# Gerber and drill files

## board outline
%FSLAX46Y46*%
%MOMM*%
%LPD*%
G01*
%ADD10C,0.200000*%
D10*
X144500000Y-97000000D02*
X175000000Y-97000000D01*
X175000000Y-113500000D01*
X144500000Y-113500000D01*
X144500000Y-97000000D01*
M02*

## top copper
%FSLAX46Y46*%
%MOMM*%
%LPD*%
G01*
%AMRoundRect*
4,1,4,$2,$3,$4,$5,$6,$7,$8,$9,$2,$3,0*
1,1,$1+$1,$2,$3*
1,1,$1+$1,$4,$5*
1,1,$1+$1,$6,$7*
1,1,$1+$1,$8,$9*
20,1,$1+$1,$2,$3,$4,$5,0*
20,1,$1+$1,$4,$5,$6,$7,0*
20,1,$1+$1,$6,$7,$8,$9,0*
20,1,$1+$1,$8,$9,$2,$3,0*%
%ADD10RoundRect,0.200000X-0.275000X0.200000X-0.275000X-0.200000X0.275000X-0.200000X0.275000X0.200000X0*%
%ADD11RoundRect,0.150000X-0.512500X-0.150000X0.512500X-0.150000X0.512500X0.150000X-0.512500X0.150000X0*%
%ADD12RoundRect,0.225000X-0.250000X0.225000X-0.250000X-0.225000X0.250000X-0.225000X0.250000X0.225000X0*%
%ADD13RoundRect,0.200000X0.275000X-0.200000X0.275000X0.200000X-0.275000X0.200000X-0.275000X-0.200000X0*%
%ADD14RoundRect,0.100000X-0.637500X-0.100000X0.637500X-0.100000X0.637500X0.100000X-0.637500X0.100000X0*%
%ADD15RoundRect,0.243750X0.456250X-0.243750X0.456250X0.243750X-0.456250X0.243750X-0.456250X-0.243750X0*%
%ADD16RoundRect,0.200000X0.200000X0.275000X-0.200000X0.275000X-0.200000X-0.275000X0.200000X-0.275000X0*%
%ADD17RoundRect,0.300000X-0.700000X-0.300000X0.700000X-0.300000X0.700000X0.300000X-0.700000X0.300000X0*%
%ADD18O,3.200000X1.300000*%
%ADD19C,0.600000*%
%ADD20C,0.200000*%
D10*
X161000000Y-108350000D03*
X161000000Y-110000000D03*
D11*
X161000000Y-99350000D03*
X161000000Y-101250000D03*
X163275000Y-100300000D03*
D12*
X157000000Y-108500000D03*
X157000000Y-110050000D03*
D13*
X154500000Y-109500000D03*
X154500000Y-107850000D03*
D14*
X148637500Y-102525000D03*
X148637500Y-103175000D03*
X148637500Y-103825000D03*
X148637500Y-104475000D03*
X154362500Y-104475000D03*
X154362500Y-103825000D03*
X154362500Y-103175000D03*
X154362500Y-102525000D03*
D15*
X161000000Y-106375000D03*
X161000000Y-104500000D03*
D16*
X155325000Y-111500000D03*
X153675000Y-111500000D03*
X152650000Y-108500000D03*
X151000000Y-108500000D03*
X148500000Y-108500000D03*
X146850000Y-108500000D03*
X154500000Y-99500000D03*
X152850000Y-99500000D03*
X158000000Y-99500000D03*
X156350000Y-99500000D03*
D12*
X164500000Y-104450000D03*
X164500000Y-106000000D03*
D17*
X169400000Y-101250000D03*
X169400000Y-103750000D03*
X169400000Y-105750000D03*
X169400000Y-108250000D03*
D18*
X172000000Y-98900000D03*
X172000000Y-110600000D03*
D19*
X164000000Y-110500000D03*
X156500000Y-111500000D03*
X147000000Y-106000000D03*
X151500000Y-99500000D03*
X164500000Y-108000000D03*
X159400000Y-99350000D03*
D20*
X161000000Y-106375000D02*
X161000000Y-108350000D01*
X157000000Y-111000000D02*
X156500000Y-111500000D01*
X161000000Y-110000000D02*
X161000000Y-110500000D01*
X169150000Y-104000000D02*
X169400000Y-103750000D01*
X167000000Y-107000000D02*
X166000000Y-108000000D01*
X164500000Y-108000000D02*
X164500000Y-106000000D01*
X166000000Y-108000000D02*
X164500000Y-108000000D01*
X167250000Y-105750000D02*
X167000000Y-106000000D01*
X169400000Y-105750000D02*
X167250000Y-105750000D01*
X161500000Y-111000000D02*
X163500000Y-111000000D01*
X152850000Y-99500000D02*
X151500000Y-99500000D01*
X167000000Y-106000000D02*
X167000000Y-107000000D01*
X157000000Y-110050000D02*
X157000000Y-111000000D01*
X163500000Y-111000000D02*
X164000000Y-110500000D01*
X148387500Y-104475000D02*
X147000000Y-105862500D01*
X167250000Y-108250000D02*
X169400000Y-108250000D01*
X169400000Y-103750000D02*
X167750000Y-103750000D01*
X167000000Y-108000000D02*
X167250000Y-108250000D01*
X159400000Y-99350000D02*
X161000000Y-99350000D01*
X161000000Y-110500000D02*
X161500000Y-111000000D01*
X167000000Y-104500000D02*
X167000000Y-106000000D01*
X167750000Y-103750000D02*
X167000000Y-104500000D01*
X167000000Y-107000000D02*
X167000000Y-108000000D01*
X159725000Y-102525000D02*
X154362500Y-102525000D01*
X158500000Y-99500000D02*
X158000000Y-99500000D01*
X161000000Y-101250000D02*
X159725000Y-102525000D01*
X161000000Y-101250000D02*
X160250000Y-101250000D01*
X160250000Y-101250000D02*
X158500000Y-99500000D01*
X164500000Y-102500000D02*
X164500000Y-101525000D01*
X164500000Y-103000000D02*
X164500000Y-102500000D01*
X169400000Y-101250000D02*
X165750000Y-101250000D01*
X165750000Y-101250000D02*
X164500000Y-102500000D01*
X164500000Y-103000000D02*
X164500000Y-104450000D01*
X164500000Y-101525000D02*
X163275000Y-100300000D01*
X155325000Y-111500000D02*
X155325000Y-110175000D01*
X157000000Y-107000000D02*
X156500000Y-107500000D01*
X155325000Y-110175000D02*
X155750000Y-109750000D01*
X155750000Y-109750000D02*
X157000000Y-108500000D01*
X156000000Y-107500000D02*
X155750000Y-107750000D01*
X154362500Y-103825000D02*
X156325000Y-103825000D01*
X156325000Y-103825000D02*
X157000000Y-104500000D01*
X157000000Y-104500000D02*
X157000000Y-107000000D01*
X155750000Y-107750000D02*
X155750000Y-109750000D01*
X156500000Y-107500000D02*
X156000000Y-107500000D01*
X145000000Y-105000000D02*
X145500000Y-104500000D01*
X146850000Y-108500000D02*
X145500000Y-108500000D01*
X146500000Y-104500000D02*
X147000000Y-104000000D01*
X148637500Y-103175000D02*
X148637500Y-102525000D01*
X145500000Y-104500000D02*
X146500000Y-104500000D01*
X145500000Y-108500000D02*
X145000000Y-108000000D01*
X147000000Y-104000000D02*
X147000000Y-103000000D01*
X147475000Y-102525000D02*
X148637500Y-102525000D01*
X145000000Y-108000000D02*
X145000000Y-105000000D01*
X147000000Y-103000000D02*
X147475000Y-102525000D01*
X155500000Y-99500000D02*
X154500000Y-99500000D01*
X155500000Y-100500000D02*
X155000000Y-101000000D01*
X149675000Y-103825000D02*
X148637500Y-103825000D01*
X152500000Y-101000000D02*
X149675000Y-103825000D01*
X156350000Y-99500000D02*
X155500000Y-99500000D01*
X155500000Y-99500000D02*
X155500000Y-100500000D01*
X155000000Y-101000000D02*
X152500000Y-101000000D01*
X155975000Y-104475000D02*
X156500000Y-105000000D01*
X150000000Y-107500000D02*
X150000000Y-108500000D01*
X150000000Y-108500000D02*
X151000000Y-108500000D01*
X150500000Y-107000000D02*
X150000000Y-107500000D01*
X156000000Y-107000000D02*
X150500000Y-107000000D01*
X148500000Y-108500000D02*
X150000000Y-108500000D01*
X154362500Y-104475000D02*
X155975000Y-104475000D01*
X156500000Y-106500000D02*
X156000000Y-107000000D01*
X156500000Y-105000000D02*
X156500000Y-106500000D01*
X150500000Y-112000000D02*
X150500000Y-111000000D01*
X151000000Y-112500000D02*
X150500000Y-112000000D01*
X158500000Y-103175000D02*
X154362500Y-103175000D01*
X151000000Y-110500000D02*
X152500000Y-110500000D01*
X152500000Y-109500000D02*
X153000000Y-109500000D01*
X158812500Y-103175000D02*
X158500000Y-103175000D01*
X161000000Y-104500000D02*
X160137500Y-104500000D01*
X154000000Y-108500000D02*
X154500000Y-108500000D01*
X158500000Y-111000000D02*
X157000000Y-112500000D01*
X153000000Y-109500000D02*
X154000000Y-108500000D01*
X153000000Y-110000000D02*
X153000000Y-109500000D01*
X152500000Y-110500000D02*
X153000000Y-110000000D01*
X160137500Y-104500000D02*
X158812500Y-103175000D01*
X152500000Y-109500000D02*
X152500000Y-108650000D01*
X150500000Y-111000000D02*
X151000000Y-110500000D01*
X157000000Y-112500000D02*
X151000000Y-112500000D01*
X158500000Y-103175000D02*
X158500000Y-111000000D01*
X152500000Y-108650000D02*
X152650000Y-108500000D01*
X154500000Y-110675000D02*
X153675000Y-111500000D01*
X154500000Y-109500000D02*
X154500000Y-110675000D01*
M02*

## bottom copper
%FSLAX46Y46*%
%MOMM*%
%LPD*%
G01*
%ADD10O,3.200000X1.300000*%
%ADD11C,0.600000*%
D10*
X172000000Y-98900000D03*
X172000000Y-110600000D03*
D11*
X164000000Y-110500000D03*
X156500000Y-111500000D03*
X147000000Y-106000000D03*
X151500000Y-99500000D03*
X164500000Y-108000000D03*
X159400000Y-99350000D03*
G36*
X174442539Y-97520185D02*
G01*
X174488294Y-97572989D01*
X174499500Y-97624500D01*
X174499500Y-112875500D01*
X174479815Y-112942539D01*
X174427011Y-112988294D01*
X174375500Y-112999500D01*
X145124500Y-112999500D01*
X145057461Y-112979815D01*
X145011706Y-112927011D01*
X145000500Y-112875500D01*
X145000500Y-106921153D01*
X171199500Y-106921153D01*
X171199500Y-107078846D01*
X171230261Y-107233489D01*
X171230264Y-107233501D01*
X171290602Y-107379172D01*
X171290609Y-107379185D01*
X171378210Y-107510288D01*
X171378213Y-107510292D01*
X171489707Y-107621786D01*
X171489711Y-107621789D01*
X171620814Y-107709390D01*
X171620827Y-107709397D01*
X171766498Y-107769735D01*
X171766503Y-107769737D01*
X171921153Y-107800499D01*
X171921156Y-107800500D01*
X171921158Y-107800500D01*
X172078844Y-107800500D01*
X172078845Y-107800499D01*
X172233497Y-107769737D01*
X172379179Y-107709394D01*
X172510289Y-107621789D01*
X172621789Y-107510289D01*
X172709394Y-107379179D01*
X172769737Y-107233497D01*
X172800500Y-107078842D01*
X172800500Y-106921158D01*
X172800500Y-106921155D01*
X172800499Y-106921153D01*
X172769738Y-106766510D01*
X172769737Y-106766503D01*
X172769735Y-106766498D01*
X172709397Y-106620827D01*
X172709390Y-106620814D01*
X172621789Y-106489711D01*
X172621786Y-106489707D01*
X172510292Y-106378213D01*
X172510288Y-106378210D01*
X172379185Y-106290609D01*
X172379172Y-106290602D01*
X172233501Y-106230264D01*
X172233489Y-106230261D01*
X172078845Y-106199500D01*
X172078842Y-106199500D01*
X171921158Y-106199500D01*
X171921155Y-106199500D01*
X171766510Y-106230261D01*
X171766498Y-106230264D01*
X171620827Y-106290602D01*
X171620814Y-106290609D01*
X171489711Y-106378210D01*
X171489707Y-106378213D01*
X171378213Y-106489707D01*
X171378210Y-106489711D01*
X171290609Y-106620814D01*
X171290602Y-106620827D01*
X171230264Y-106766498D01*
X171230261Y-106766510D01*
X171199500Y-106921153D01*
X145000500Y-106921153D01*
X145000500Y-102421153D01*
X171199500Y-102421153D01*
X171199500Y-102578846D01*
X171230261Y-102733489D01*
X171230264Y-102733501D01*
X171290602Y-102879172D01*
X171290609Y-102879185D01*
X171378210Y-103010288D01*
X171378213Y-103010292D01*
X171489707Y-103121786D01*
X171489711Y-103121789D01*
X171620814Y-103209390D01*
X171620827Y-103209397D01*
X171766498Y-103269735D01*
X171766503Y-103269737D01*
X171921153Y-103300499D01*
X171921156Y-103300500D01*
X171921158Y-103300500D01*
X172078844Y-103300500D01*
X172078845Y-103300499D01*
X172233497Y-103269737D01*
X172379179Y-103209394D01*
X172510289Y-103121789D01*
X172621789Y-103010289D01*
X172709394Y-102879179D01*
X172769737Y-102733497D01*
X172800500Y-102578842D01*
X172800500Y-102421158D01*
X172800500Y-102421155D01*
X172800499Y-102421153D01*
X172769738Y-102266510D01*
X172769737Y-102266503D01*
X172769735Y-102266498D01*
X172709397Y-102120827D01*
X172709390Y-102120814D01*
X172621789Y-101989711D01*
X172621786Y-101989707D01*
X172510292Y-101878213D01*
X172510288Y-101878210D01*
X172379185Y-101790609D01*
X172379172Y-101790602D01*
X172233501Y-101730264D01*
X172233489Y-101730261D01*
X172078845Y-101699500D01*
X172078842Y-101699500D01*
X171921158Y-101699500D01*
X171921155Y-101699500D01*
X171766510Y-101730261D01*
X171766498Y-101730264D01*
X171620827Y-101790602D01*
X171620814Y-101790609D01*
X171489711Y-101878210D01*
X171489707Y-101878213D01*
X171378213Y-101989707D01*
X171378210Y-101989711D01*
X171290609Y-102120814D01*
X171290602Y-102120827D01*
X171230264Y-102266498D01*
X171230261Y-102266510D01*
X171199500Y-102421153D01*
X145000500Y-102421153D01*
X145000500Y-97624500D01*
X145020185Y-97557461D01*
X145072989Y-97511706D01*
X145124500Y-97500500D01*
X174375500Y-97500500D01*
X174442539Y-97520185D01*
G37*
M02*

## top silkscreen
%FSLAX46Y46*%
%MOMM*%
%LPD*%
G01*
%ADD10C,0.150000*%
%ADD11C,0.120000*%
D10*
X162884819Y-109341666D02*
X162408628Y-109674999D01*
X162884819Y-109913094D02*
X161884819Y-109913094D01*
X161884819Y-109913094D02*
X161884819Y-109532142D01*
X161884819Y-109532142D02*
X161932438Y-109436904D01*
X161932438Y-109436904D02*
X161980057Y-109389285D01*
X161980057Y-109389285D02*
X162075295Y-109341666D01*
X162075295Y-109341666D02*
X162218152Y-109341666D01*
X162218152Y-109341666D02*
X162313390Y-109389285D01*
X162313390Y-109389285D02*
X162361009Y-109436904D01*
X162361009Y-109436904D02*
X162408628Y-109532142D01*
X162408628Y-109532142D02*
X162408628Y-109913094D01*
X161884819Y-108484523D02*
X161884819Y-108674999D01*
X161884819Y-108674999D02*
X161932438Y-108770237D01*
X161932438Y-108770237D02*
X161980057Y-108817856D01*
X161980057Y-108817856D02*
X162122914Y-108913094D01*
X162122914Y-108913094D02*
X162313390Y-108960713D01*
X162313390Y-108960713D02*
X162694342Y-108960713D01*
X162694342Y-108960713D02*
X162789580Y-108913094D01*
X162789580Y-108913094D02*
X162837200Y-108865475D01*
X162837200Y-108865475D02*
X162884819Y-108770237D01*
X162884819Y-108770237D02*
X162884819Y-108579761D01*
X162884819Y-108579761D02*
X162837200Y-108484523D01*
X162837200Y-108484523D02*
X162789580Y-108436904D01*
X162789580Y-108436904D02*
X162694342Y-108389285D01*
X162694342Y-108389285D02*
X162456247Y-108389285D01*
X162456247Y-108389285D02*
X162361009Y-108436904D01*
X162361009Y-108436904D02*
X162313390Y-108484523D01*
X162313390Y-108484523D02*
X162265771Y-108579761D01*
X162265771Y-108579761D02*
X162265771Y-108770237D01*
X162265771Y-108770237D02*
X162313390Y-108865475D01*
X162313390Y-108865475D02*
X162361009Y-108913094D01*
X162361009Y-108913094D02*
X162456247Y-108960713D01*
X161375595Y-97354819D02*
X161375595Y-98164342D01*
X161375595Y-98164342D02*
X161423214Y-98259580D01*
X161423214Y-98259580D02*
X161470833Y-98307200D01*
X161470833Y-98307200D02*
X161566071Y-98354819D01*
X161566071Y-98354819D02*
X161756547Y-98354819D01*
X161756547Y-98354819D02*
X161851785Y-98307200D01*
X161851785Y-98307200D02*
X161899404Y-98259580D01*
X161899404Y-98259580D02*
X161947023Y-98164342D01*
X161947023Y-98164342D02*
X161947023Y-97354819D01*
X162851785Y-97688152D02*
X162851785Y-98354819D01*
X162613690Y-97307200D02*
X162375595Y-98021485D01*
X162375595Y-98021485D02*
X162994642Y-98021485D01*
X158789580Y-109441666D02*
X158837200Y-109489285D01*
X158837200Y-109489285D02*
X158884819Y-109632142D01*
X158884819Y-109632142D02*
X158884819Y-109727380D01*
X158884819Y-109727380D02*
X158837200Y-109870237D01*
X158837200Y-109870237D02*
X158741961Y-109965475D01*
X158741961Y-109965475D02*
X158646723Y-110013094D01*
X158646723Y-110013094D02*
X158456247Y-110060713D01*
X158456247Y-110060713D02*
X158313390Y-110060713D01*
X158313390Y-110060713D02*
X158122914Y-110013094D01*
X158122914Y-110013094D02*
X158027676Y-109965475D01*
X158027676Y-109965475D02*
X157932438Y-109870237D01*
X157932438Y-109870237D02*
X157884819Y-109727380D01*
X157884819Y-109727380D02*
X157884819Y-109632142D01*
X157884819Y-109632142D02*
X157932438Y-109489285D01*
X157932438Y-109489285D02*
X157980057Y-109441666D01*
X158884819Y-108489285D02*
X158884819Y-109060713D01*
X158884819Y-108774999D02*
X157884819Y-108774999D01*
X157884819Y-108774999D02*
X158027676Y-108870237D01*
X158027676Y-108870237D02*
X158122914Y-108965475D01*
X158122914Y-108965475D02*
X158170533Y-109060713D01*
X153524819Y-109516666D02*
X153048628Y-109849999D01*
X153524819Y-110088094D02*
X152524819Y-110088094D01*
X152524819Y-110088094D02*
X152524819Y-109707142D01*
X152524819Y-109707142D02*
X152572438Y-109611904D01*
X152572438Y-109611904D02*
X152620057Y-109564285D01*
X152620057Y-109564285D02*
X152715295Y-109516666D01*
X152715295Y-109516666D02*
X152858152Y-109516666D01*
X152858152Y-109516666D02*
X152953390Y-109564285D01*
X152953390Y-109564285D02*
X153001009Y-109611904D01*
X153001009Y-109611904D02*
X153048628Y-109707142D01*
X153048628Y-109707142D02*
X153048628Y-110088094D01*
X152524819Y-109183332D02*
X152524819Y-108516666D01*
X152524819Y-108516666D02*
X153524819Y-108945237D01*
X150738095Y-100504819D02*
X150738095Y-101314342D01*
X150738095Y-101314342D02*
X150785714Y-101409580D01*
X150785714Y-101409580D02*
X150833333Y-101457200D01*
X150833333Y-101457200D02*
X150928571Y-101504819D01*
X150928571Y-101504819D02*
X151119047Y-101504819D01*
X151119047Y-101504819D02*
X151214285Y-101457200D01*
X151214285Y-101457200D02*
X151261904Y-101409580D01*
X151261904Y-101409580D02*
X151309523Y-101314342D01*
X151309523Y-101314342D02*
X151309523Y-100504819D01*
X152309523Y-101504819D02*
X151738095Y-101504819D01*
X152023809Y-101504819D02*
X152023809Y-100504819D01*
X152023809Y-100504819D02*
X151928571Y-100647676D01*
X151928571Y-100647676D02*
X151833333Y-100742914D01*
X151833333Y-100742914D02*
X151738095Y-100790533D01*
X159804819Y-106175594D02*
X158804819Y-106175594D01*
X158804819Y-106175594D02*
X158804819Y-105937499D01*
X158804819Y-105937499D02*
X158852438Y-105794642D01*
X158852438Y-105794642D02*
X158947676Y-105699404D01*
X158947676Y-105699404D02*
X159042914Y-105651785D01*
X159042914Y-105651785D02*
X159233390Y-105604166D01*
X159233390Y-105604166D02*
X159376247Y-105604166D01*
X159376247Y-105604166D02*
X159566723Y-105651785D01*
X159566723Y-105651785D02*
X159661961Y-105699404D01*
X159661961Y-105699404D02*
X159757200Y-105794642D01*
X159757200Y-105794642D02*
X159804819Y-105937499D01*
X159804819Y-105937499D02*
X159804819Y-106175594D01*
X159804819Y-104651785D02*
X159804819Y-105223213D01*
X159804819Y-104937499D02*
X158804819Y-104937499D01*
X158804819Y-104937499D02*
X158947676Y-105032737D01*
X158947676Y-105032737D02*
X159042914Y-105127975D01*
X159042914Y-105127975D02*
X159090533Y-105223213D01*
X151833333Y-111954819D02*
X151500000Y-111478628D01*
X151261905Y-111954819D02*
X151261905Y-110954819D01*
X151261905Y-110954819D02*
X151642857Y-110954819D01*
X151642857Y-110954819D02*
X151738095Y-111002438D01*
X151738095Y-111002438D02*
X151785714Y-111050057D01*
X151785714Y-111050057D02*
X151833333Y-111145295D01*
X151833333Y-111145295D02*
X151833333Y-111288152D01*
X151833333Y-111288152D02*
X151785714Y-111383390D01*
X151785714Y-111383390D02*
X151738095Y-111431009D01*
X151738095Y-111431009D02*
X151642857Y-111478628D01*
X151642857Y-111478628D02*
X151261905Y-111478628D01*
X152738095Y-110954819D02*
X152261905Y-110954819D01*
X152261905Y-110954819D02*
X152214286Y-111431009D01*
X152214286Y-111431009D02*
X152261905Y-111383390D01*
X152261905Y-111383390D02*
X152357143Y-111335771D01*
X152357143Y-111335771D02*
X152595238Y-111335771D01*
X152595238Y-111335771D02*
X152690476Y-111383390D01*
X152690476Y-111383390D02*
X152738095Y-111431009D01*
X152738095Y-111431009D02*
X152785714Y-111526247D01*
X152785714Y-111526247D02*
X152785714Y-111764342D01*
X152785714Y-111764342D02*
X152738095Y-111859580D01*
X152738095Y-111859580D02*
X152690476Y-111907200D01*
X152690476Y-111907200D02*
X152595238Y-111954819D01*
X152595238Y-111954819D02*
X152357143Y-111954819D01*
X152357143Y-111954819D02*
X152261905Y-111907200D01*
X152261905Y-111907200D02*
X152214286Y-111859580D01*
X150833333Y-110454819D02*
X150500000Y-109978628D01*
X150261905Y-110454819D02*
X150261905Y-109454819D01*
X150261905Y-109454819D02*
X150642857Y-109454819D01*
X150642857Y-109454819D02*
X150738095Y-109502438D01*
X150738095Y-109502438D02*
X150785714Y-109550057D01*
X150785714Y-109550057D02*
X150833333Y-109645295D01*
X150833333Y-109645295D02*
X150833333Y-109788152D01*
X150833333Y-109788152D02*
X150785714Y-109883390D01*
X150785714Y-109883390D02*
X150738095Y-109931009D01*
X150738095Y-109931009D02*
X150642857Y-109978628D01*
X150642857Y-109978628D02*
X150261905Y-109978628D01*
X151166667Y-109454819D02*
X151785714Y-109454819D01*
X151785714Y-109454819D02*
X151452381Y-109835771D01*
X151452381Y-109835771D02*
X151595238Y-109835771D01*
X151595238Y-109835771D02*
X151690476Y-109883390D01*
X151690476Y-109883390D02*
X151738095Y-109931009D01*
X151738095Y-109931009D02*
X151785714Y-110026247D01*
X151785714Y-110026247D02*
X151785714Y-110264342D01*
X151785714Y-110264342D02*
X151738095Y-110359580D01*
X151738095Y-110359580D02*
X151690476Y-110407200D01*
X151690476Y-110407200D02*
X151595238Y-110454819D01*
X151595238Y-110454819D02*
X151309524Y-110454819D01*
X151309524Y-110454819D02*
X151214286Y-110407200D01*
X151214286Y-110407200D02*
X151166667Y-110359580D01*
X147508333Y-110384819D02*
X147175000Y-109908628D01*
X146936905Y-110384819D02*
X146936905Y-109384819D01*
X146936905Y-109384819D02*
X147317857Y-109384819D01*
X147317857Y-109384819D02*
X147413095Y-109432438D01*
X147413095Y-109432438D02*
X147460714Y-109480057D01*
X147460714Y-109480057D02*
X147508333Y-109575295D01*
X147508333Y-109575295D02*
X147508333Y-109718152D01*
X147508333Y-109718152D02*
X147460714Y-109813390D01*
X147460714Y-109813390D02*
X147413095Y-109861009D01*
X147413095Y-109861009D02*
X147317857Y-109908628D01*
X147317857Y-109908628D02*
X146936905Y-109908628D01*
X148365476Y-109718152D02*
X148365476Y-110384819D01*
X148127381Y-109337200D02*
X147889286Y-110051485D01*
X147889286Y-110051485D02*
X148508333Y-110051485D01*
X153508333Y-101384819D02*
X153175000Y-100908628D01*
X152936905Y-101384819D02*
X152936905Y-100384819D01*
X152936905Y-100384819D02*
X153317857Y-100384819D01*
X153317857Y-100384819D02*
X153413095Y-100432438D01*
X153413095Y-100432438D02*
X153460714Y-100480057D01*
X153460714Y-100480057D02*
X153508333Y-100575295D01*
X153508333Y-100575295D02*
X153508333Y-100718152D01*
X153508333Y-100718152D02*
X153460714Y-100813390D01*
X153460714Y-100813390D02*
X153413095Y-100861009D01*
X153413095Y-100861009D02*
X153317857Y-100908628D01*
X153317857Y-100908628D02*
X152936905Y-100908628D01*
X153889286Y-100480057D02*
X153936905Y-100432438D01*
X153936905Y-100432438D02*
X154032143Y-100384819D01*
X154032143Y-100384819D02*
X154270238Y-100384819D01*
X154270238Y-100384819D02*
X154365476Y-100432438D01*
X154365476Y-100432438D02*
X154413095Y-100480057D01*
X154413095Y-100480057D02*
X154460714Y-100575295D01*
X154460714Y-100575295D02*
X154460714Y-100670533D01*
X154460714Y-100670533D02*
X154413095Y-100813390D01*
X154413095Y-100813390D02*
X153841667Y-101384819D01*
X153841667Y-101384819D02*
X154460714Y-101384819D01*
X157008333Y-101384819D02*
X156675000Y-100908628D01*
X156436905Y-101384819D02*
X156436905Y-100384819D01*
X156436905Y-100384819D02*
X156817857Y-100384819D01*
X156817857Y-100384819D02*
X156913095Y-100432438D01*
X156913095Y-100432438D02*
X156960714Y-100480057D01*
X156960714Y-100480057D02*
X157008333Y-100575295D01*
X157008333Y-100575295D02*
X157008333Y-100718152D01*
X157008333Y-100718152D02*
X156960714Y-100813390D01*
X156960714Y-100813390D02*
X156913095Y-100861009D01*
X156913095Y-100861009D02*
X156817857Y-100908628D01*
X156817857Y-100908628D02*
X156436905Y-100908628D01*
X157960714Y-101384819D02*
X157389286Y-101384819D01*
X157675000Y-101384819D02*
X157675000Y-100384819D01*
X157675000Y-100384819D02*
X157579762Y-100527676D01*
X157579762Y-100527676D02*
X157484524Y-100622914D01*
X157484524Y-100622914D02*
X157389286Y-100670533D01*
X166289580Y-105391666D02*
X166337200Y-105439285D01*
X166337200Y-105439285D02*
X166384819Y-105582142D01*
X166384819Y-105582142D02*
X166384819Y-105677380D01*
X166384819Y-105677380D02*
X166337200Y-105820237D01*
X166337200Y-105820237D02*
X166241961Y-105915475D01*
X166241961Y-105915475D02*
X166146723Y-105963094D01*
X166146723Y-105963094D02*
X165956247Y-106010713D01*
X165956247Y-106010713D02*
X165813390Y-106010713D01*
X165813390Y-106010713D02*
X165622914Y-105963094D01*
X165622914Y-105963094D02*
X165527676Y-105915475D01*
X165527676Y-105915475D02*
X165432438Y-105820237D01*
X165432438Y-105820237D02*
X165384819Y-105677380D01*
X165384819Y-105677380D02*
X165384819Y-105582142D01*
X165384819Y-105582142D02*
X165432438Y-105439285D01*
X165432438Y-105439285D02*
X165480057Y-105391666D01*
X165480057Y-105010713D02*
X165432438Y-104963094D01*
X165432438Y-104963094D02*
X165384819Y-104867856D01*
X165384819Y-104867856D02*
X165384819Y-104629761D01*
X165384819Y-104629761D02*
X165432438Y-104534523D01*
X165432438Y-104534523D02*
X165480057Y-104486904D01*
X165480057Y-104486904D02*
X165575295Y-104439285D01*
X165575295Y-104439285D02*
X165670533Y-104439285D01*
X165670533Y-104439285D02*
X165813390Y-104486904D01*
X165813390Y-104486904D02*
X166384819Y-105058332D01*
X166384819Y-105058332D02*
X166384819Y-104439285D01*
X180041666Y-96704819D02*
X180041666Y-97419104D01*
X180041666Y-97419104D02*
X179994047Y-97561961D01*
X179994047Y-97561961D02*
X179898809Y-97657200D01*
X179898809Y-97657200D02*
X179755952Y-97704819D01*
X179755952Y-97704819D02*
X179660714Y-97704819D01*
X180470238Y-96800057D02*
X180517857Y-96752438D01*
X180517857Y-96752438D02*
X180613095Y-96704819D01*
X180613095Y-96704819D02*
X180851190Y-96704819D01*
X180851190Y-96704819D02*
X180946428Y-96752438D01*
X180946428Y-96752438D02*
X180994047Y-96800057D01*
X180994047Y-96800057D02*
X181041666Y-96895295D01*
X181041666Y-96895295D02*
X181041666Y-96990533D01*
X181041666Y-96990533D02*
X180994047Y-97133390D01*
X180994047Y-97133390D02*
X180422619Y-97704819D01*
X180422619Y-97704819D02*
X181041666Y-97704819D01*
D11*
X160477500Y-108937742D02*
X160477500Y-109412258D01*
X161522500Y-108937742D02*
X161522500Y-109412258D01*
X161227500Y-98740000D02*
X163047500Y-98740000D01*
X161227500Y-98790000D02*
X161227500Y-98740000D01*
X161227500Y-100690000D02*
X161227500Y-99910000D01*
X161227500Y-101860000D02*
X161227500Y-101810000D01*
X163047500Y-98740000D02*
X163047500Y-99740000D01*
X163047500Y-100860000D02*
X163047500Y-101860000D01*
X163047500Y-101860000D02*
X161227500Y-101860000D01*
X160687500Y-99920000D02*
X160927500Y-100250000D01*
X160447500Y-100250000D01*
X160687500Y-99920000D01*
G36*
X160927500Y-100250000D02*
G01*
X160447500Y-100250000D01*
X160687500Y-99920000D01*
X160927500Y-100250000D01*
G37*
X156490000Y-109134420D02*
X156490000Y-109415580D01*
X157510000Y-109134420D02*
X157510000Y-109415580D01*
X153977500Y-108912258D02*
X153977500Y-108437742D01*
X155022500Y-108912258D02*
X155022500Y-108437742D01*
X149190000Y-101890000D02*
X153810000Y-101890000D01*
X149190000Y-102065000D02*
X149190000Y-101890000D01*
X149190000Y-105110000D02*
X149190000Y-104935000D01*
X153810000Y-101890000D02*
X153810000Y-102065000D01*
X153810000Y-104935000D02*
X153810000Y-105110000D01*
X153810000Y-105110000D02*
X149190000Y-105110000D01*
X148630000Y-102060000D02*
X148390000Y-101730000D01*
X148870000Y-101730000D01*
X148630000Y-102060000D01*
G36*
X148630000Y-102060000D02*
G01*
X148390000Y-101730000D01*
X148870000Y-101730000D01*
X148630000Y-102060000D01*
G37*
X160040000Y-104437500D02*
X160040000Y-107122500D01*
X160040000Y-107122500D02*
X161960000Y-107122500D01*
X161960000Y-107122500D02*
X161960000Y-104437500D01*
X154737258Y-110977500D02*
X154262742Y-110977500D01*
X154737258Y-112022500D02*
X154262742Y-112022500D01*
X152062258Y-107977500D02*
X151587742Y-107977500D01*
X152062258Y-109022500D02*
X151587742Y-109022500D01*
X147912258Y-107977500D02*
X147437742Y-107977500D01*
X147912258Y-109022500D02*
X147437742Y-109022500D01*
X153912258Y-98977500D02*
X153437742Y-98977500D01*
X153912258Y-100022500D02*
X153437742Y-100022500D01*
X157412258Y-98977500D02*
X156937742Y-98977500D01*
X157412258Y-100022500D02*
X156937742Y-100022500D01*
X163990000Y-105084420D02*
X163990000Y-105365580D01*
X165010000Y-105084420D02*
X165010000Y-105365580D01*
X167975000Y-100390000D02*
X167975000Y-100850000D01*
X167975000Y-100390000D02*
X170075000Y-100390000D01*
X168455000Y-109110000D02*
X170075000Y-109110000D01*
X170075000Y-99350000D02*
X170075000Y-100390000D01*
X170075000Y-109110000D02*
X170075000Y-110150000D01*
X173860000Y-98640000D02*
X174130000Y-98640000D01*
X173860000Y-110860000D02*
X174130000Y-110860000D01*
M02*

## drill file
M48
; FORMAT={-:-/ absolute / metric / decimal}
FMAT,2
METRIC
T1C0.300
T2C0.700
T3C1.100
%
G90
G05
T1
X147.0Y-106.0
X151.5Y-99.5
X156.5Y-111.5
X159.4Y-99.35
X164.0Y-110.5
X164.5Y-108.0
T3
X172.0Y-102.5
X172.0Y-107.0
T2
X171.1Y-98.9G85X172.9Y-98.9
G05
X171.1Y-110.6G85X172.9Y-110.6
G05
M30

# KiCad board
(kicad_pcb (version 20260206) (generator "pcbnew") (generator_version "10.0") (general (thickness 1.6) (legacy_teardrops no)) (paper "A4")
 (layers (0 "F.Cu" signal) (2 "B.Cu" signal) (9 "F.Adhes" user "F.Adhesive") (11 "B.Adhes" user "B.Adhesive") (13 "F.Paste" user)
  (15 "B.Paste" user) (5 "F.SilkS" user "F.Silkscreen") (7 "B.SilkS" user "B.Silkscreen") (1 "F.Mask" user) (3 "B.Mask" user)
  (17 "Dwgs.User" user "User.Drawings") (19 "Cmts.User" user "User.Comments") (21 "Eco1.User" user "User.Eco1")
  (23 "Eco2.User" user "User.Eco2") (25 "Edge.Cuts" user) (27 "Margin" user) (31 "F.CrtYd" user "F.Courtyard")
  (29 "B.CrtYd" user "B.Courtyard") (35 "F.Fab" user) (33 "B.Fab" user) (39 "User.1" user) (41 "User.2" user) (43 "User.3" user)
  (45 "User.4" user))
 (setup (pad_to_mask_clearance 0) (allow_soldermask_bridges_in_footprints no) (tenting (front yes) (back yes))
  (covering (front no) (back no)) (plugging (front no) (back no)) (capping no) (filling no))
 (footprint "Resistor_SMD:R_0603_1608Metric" (layer "F.Cu") (at 161 109.175 -90)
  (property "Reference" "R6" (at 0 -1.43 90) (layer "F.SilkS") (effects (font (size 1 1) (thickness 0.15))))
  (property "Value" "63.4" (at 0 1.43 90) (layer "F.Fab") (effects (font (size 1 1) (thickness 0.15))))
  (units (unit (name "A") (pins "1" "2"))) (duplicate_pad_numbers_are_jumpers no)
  (fp_line (start -0.237258 0.5225) (end 0.237258 0.5225) (stroke (width 0.12) (type solid)) (layer "F.SilkS"))
  (fp_line (start -0.237258 -0.5225) (end 0.237258 -0.5225) (stroke (width 0.12) (type solid)) (layer "F.SilkS"))
  (pad "1" smd roundrect (at -0.825 0 270) (size 0.8 0.95) (layers "F.Cu" "F.Mask" "F.Paste") (roundrect_rratio 0.25) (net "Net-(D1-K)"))
  (pad "2" smd roundrect (at 0.825 0 270) (size 0.8 0.95) (layers "F.Cu" "F.Mask" "F.Paste") (roundrect_rratio 0.25) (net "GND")))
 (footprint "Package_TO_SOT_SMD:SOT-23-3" (layer "F.Cu") (at 162.1375 100.3)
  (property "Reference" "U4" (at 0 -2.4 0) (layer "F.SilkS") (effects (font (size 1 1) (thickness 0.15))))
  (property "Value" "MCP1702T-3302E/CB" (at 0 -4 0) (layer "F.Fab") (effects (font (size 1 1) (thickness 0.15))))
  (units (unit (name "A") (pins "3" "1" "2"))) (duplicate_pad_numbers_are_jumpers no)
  (fp_line (start -0.91 -1.56) (end 0.91 -1.56) (stroke (width 0.12) (type solid)) (layer "F.SilkS"))
  (fp_line (start -0.91 -1.51) (end -0.91 -1.56) (stroke (width 0.12) (type solid)) (layer "F.SilkS"))
  (fp_line (start -0.91 0.39) (end -0.91 -0.39) (stroke (width 0.12) (type solid)) (layer "F.SilkS"))
  (fp_line (start -0.91 1.56) (end -0.91 1.51) (stroke (width 0.12) (type solid)) (layer "F.SilkS"))
  (fp_line (start 0.91 -1.56) (end 0.91 -0.56) (stroke (width 0.12) (type solid)) (layer "F.SilkS"))
  (fp_line (start 0.91 0.56) (end 0.91 1.56) (stroke (width 0.12) (type solid)) (layer "F.SilkS"))
  (fp_line (start 0.91 1.56) (end -0.91 1.56) (stroke (width 0.12) (type solid)) (layer "F.SilkS"))
  (fp_poly (pts (xy -1.45 -0.38) (xy -1.21 -0.05) (xy -1.69 -0.05)) (stroke (width 0.12) (type solid)) (fill yes) (layer "F.SilkS"))
  (pad "1" smd roundrect (at -1.1375 -0.95) (size 1.325 0.6) (layers "F.Cu" "F.Mask" "F.Paste") (roundrect_rratio 0.25) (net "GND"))
  (pad "2" smd roundrect (at -1.1375 0.95) (size 1.325 0.6) (layers "F.Cu" "F.Mask" "F.Paste") (roundrect_rratio 0.25) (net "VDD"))
  (pad "3" smd roundrect (at 1.1375 0) (size 1.325 0.6) (layers "F.Cu" "F.Mask" "F.Paste") (roundrect_rratio 0.25) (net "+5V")))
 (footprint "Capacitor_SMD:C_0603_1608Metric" (layer "F.Cu") (at 157 109.275 -90)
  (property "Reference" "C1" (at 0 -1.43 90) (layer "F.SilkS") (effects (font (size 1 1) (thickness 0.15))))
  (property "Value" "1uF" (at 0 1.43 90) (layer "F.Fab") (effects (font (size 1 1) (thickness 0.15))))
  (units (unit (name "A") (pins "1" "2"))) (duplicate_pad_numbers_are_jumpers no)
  (fp_line (start -0.14058 0.51) (end 0.14058 0.51) (stroke (width 0.12) (type solid)) (layer "F.SilkS"))
  (fp_line (start -0.14058 -0.51) (end 0.14058 -0.51) (stroke (width 0.12) (type solid)) (layer "F.SilkS"))
  (pad "1" smd roundrect (at -0.775 0 270) (size 0.9 0.95) (layers "F.Cu" "F.Mask" "F.Paste") (roundrect_rratio 0.25) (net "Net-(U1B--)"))
  (pad "2" smd roundrect (at 0.775 0 270) (size 0.9 0.95) (layers "F.Cu" "F.Mask" "F.Paste") (roundrect_rratio 0.25) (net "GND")))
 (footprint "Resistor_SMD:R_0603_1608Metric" (layer "F.Cu") (at 154.5 108.675 90)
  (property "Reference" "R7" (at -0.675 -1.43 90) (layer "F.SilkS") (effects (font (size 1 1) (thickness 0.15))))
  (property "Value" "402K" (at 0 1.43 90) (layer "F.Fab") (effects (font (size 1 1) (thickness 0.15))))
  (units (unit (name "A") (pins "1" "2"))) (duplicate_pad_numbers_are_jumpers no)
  (fp_line (start -0.237258 -0.5225) (end 0.237258 -0.5225) (stroke (width 0.12) (type solid)) (layer "F.SilkS"))
  (fp_line (start -0.237258 0.5225) (end 0.237258 0.5225) (stroke (width 0.12) (type solid)) (layer "F.SilkS"))
  (pad "1" smd roundrect (at -0.825 0 90) (size 0.8 0.95) (layers "F.Cu" "F.Mask" "F.Paste") (roundrect_rratio 0.25) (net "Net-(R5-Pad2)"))
  (pad "2" smd roundrect (at 0.825 0 90) (size 0.8 0.95) (layers "F.Cu" "F.Mask" "F.Paste") (roundrect_rratio 0.25) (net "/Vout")))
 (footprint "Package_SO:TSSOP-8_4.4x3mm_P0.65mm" (layer "F.Cu") (at 151.5 103.5)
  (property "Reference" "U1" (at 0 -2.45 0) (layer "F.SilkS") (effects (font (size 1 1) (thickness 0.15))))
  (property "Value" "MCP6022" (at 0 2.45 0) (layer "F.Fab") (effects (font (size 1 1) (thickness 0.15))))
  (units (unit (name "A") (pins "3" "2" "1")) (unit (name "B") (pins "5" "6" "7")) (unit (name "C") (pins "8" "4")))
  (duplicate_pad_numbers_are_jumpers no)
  (fp_line (start -2.31 -1.61) (end 2.31 -1.61) (stroke (width 0.12) (type solid)) (layer "F.SilkS"))
  (fp_line (start -2.31 -1.435) (end -2.31 -1.61) (stroke (width 0.12) (type solid)) (layer "F.SilkS"))
  (fp_line (start -2.31 1.61) (end -2.31 1.435) (stroke (width 0.12) (type solid)) (layer "F.SilkS"))
  (fp_line (start 2.31 -1.61) (end 2.31 -1.435) (stroke (width 0.12) (type solid)) (layer "F.SilkS"))
  (fp_line (start 2.31 1.435) (end 2.31 1.61) (stroke (width 0.12) (type solid)) (layer "F.SilkS"))
  (fp_line (start 2.31 1.61) (end -2.31 1.61) (stroke (width 0.12) (type solid)) (layer "F.SilkS"))
  (fp_poly (pts (xy -2.87 -1.44) (xy -3.11 -1.77) (xy -2.63 -1.77)) (stroke (width 0.12) (type solid)) (fill yes) (layer "F.SilkS"))
  (pad "1" smd roundrect (at -2.8625 -0.975) (size 1.475 0.4) (layers "F.Cu" "F.Mask" "F.Paste") (roundrect_rratio 0.25) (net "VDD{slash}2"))
  (pad "2" smd roundrect (at -2.8625 -0.325) (size 1.475 0.4) (layers "F.Cu" "F.Mask" "F.Paste") (roundrect_rratio 0.25) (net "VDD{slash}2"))
  (pad "3" smd roundrect (at -2.8625 0.325) (size 1.475 0.4) (layers "F.Cu" "F.Mask" "F.Paste") (roundrect_rratio 0.25) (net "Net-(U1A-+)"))
  (pad "4" smd roundrect (at -2.8625 0.975) (size 1.475 0.4) (layers "F.Cu" "F.Mask" "F.Paste") (roundrect_rratio 0.25) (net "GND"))
  (pad "5" smd roundrect (at 2.8625 0.975) (size 1.475 0.4) (layers "F.Cu" "F.Mask" "F.Paste") (roundrect_rratio 0.25) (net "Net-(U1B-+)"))
  (pad "6" smd roundrect (at 2.8625 0.325) (size 1.475 0.4) (layers "F.Cu" "F.Mask" "F.Paste") (roundrect_rratio 0.25) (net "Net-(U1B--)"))
  (pad "7" smd roundrect (at 2.8625 -0.325) (size 1.475 0.4) (layers "F.Cu" "F.Mask" "F.Paste") (roundrect_rratio 0.25) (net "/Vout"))
  (pad "8" smd roundrect (at 2.8625 -0.975) (size 1.475 0.4) (layers "F.Cu" "F.Mask" "F.Paste") (roundrect_rratio 0.25) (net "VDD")))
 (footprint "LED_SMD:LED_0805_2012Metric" (layer "F.Cu") (at 161 105.4375 90)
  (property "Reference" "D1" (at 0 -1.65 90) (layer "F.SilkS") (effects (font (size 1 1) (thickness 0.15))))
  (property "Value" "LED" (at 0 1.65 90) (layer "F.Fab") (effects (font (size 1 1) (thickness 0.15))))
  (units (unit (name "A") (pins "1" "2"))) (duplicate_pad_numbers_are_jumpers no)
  (fp_line (start 1 -0.96) (end -1.685 -0.96) (stroke (width 0.12) (type solid)) (layer "F.SilkS"))
  (fp_line (start -1.685 -0.96) (end -1.685 0.96) (stroke (width 0.12) (type solid)) (layer "F.SilkS"))
  (fp_line (start -1.685 0.96) (end 1 0.96) (stroke (width 0.12) (type solid)) (layer "F.SilkS"))
  (pad "1" smd roundrect (at -0.9375 0 90) (size 0.975 1.4) (layers "F.Cu" "F.Mask" "F.Paste") (roundrect_rratio 0.25) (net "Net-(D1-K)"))
  (pad "2" smd roundrect (at 0.9375 0 90) (size 0.975 1.4) (layers "F.Cu" "F.Mask" "F.Paste") (roundrect_rratio 0.25) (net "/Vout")))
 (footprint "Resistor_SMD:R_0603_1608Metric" (layer "F.Cu") (at 154.5 111.5 180)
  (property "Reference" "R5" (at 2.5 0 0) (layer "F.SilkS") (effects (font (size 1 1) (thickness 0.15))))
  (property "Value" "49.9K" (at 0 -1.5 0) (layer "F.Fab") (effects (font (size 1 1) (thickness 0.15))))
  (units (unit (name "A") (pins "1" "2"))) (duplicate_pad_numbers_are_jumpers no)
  (fp_line (start -0.237258 0.5225) (end 0.237258 0.5225) (stroke (width 0.12) (type solid)) (layer "F.SilkS"))
  (fp_line (start -0.237258 -0.5225) (end 0.237258 -0.5225) (stroke (width 0.12) (type solid)) (layer "F.SilkS"))
  (pad "1" smd roundrect (at -0.825 0 180) (size 0.8 0.95) (layers "F.Cu" "F.Mask" "F.Paste") (roundrect_rratio 0.25) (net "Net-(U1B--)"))
  (pad "2" smd roundrect (at 0.825 0 180) (size 0.8 0.95) (layers "F.Cu" "F.Mask" "F.Paste") (roundrect_rratio 0.25) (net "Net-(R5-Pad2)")))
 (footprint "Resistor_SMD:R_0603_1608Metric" (layer "F.Cu") (at 151.825 108.5 180)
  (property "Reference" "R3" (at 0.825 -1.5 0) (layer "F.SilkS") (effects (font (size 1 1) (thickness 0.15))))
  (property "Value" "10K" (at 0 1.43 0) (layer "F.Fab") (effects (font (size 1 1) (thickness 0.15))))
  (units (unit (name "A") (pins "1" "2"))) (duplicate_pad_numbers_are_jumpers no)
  (fp_line (start -0.237258 0.5225) (end 0.237258 0.5225) (stroke (width 0.12) (type solid)) (layer "F.SilkS"))
  (fp_line (start -0.237258 -0.5225) (end 0.237258 -0.5225) (stroke (width 0.12) (type solid)) (layer "F.SilkS"))
  (pad "1" smd roundrect (at -0.825 0 180) (size 0.8 0.95) (layers "F.Cu" "F.Mask" "F.Paste") (roundrect_rratio 0.25) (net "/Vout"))
  (pad "2" smd roundrect (at 0.825 0 180) (size 0.8 0.95) (layers "F.Cu" "F.Mask" "F.Paste") (roundrect_rratio 0.25) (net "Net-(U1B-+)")))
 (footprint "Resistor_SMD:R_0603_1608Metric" (layer "F.Cu") (at 147.675 108.5 180)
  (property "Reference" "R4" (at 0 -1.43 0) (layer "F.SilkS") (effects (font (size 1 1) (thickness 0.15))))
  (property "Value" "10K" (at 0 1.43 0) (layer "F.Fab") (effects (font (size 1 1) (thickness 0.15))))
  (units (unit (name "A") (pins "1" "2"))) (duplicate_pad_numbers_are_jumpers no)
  (fp_line (start -0.237258 0.5225) (end 0.237258 0.5225) (stroke (width 0.12) (type solid)) (layer "F.SilkS"))
  (fp_line (start -0.237258 -0.5225) (end 0.237258 -0.5225) (stroke (width 0.12) (type solid)) (layer "F.SilkS"))
  (pad "1" smd roundrect (at -0.825 0 180) (size 0.8 0.95) (layers "F.Cu" "F.Mask" "F.Paste") (roundrect_rratio 0.25) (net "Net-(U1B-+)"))
  (pad "2" smd roundrect (at 0.825 0 180) (size 0.8 0.95) (layers "F.Cu" "F.Mask" "F.Paste") (roundrect_rratio 0.25) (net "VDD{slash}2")))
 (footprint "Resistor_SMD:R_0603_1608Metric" (layer "F.Cu") (at 153.675 99.5 180)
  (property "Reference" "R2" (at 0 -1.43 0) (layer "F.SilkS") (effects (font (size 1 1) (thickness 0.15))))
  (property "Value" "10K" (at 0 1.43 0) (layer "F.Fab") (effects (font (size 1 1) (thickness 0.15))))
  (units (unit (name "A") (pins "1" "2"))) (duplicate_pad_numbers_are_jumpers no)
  (fp_line (start -0.237258 0.5225) (end 0.237258 0.5225) (stroke (width 0.12) (type solid)) (layer "F.SilkS"))
  (fp_line (start -0.237258 -0.5225) (end 0.237258 -0.5225) (stroke (width 0.12) (type solid)) (layer "F.SilkS"))
  (pad "1" smd roundrect (at -0.825 0 180) (size 0.8 0.95) (layers "F.Cu" "F.Mask" "F.Paste") (roundrect_rratio 0.25) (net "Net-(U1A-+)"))
  (pad "2" smd roundrect (at 0.825 0 180) (size 0.8 0.95) (layers "F.Cu" "F.Mask" "F.Paste") (roundrect_rratio 0.25) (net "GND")))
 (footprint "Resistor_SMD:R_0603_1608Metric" (layer "F.Cu") (at 157.175 99.5 180)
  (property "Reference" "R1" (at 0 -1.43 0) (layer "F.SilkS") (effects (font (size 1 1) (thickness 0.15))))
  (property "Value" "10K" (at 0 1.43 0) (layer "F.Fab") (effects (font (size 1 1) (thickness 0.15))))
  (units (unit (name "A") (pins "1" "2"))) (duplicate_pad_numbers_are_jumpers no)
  (fp_line (start -0.237258 0.5225) (end 0.237258 0.5225) (stroke (width 0.12) (type solid)) (layer "F.SilkS"))
  (fp_line (start -0.237258 -0.5225) (end 0.237258 -0.5225) (stroke (width 0.12) (type solid)) (layer "F.SilkS"))
  (pad "1" smd roundrect (at -0.825 0 180) (size 0.8 0.95) (layers "F.Cu" "F.Mask" "F.Paste") (roundrect_rratio 0.25) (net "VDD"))
  (pad "2" smd roundrect (at 0.825 0 180) (size 0.8 0.95) (layers "F.Cu" "F.Mask" "F.Paste") (roundrect_rratio 0.25) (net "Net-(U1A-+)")))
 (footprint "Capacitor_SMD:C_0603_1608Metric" (layer "F.Cu") (at 164.5 105.225 -90)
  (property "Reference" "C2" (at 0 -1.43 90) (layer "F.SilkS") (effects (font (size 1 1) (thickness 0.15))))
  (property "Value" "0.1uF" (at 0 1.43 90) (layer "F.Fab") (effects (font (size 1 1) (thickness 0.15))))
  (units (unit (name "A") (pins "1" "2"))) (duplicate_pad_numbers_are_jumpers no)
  (fp_line (start -0.14058 0.51) (end 0.14058 0.51) (stroke (width 0.12) (type solid)) (layer "F.SilkS"))
  (fp_line (start -0.14058 -0.51) (end 0.14058 -0.51) (stroke (width 0.12) (type solid)) (layer "F.SilkS"))
  (pad "1" smd roundrect (at -0.775 0 270) (size 0.9 0.95) (layers "F.Cu" "F.Mask" "F.Paste") (roundrect_rratio 0.25) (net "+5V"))
  (pad "2" smd roundrect (at 0.775 0 270) (size 0.9 0.95) (layers "F.Cu" "F.Mask" "F.Paste") (roundrect_rratio 0.25) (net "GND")))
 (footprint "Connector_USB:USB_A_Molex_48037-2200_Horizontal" (layer "F.Cu") (at 180.375 104.75)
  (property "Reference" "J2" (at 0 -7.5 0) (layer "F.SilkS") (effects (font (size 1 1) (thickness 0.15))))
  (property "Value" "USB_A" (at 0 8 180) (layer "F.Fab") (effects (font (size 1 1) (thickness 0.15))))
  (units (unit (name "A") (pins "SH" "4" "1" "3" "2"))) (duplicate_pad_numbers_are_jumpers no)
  (fp_line (start -12.4 -4.36) (end -12.4 -3.9) (stroke (width 0.12) (type default)) (layer "F.SilkS"))
  (fp_line (start -12.4 -4.36) (end -10.3 -4.36) (stroke (width 0.12) (type default)) (layer "F.SilkS"))
  (fp_line (start -11.92 4.36) (end -10.3 4.36) (stroke (width 0.12) (type default)) (layer "F.SilkS"))
  (fp_line (start -10.3 -5.4) (end -10.3 -4.36) (stroke (width 0.12) (type default)) (layer "F.SilkS"))
  (fp_line (start -10.3 4.36) (end -10.3 5.4) (stroke (width 0.12) (type default)) (layer "F.SilkS"))
  (fp_line (start -6.515 -6.11) (end -6.245 -6.11) (stroke (width 0.12) (type solid)) (layer "F.SilkS"))
  (fp_line (start -6.515 6.11) (end -6.245 6.11) (stroke (width 0.12) (type solid)) (layer "F.SilkS"))
  (pad "" np_thru_hole circle (at -8.375 -2.25) (size 1.1 1.1) (drill 1.1) (layers "*.Mask"))
  (pad "" np_thru_hole circle (at -8.375 2.25) (size 1.1 1.1) (drill 1.1) (layers "*.Mask"))
  (pad "1" smd roundrect (at -10.975 -3.5) (size 2 1.2) (layers "F.Cu" "F.Mask" "F.Paste") (roundrect_rratio 0.25) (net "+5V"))
  (pad "2" smd roundrect (at -10.975 -1) (size 2 1.2) (layers "F.Cu" "F.Mask" "F.Paste") (roundrect_rratio 0.25) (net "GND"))
  (pad "3" smd roundrect (at -10.975 1) (size 2 1.2) (layers "F.Cu" "F.Mask" "F.Paste") (roundrect_rratio 0.25) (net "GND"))
  (pad "4" smd roundrect (at -10.975 3.5) (size 2 1.2) (layers "F.Cu" "F.Mask" "F.Paste") (roundrect_rratio 0.25) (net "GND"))
  (pad "SH" thru_hole oval (at -8.375 -5.85) (size 3.2 1.3) (drill oval 2.5 0.7) (layers "*.Cu" "*.Mask") (remove_unused_layers no)
   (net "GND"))
  (pad "SH" thru_hole oval (at -8.375 5.85) (size 3.2 1.3) (drill oval 2.5 0.7) (layers "*.Cu" "*.Mask") (remove_unused_layers no)
   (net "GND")))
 (gr_rect (start 144.5 97) (end 175 113.5) (stroke (width 0.2) (type default)) (fill no) (layer "Edge.Cuts"))
 (segment (start 161 106.375) (end 161 108.35) (width 0.2) (layer "F.Cu") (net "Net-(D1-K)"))
 (segment (start 157 111) (end 156.5 111.5) (width 0.2) (layer "F.Cu") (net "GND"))
 (segment (start 161 110) (end 161 110.5) (width 0.2) (layer "F.Cu") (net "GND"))
 (segment (start 169.15 104) (end 169.4 103.75) (width 0.2) (layer "F.Cu") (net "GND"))
 (segment (start 167 107) (end 166 108) (width 0.2) (layer "F.Cu") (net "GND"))
 (segment (start 164.5 108) (end 164.5 106) (width 0.2) (layer "F.Cu") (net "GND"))
 (segment (start 166 108) (end 164.5 108) (width 0.2) (layer "F.Cu") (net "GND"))
 (segment (start 167.25 105.75) (end 167 106) (width 0.2) (layer "F.Cu") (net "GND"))
 (segment (start 169.4 105.75) (end 167.25 105.75) (width 0.2) (layer "F.Cu") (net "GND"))
 (segment (start 161.5 111) (end 163.5 111) (width 0.2) (layer "F.Cu") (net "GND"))
 (segment (start 152.85 99.5) (end 151.5 99.5) (width 0.2) (layer "F.Cu") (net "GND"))
 (segment (start 167 106) (end 167 107) (width 0.2) (layer "F.Cu") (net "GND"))
 (segment (start 157 110.05) (end 157 111) (width 0.2) (layer "F.Cu") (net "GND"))
 (segment (start 163.5 111) (end 164 110.5) (width 0.2) (layer "F.Cu") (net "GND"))
 (segment (start 148.3875 104.475) (end 147 105.8625) (width 0.2) (layer "F.Cu") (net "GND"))
 (segment (start 167.25 108.25) (end 169.4 108.25) (width 0.2) (layer "F.Cu") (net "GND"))
 (segment (start 169.4 103.75) (end 167.75 103.75) (width 0.2) (layer "F.Cu") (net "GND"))
 (segment (start 167 108) (end 167.25 108.25) (width 0.2) (layer "F.Cu") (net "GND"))
 (segment (start 159.4 99.35) (end 161 99.35) (width 0.2) (layer "F.Cu") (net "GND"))
 (segment (start 161 110.5) (end 161.5 111) (width 0.2) (layer "F.Cu") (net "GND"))
 (segment (start 167 104.5) (end 167 106) (width 0.2) (layer "F.Cu") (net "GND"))
 (segment (start 167.75 103.75) (end 167 104.5) (width 0.2) (layer "F.Cu") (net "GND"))
 (segment (start 167 107) (end 167 108) (width 0.2) (layer "F.Cu") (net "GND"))
 (via (at 164 110.5) (size 0.6) (drill 0.3) (layers "F.Cu" "B.Cu") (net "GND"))
 (via (at 156.5 111.5) (size 0.6) (drill 0.3) (layers "F.Cu" "B.Cu") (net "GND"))
 (via (at 147 106) (size 0.6) (drill 0.3) (layers "F.Cu" "B.Cu") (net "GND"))
 (via (at 151.5 99.5) (size 0.6) (drill 0.3) (layers "F.Cu" "B.Cu") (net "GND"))
 (via (at 164.5 108) (size 0.6) (drill 0.3) (layers "F.Cu" "B.Cu") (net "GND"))
 (via (at 159.4 99.35) (size 0.6) (drill 0.3) (layers "F.Cu" "B.Cu") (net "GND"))
 (segment (start 159.725 102.525) (end 154.3625 102.525) (width 0.2) (layer "F.Cu") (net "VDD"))
 (segment (start 158.5 99.5) (end 158 99.5) (width 0.2) (layer "F.Cu") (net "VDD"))
 (segment (start 161 101.25) (end 159.725 102.525) (width 0.2) (layer "F.Cu") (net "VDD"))
 (segment (start 161 101.25) (end 160.25 101.25) (width 0.2) (layer "F.Cu") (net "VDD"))
 (segment (start 160.25 101.25) (end 158.5 99.5) (width 0.2) (layer "F.Cu") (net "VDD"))
 (segment (start 164.5 102.5) (end 164.5 101.525) (width 0.2) (layer "F.Cu") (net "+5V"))
 (segment (start 164.5 103) (end 164.5 102.5) (width 0.2) (layer "F.Cu") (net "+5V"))
 (segment (start 169.4 101.25) (end 165.75 101.25) (width 0.2) (layer "F.Cu") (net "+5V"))
 (segment (start 165.75 101.25) (end 164.5 102.5) (width 0.2) (layer "F.Cu") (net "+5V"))
 (segment (start 164.5 103) (end 164.5 104.45) (width 0.2) (layer "F.Cu") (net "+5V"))
 (segment (start 164.5 101.525) (end 163.275 100.3) (width 0.2) (layer "F.Cu") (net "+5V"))
 (segment (start 155.325 111.5) (end 155.325 110.175) (width 0.2) (layer "F.Cu") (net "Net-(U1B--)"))
 (segment (start 157 107) (end 156.5 107.5) (width 0.2) (layer "F.Cu") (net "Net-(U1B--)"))
 (segment (start 155.325 110.175) (end 155.75 109.75) (width 0.2) (layer "F.Cu") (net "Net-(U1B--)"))
 (segment (start 155.75 109.75) (end 157 108.5) (width 0.2) (layer "F.Cu") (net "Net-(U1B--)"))
 (segment (start 156 107.5) (end 155.75 107.75) (width 0.2) (layer "F.Cu") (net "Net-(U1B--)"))
 (segment (start 154.3625 103.825) (end 156.325 103.825) (width 0.2) (layer "F.Cu") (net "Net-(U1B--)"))
 (segment (start 156.325 103.825) (end 157 104.5) (width 0.2) (layer "F.Cu") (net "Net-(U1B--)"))
 (segment (start 157 104.5) (end 157 107) (width 0.2) (layer "F.Cu") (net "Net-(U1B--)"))
 (segment (start 155.75 107.75) (end 155.75 109.75) (width 0.2) (layer "F.Cu") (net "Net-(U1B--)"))
 (segment (start 156.5 107.5) (end 156 107.5) (width 0.2) (layer "F.Cu") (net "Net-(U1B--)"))
 (segment (start 145 105) (end 145.5 104.5) (width 0.2) (layer "F.Cu") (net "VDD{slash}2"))
 (segment (start 146.85 108.5) (end 145.5 108.5) (width 0.2) (layer "F.Cu") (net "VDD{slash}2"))
 (segment (start 146.5 104.5) (end 147 104) (width 0.2) (layer "F.Cu") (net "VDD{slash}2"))
 (segment (start 148.6375 103.175) (end 148.6375 102.525) (width 0.2) (layer "F.Cu") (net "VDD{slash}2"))
 (segment (start 145.5 104.5) (end 146.5 104.5) (width 0.2) (layer "F.Cu") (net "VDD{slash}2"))
 (segment (start 145.5 108.5) (end 145 108) (width 0.2) (layer "F.Cu") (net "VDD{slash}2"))
 (segment (start 147 104) (end 147 103) (width 0.2) (layer "F.Cu") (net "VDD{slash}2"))
 (segment (start 147.475 102.525) (end 148.6375 102.525) (width 0.2) (layer "F.Cu") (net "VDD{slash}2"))
 (segment (start 145 108) (end 145 105) (width 0.2) (layer "F.Cu") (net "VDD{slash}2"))
 (segment (start 147 103) (end 147.475 102.525) (width 0.2) (layer "F.Cu") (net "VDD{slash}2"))
 (segment (start 155.5 99.5) (end 154.5 99.5) (width 0.2) (layer "F.Cu") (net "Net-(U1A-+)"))
 (segment (start 155.5 100.5) (end 155 101) (width 0.2) (layer "F.Cu") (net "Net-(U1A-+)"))
 (segment (start 149.675 103.825) (end 148.6375 103.825) (width 0.2) (layer "F.Cu") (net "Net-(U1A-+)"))
 (segment (start 152.5 101) (end 149.675 103.825) (width 0.2) (layer "F.Cu") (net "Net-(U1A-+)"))
 (segment (start 156.35 99.5) (end 155.5 99.5) (width 0.2) (layer "F.Cu") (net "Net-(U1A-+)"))
 (segment (start 155.5 99.5) (end 155.5 100.5) (width 0.2) (layer "F.Cu") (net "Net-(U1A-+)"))
 (segment (start 155 101) (end 152.5 101) (width 0.2) (layer "F.Cu") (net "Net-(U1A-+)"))
 (segment (start 155.975 104.475) (end 156.5 105) (width 0.2) (layer "F.Cu") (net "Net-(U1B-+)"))
 (segment (start 150 107.5) (end 150 108.5) (width 0.2) (layer "F.Cu") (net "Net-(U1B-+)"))
 (segment (start 150 108.5) (end 151 108.5) (width 0.2) (layer "F.Cu") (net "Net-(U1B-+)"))
 (segment (start 150.5 107) (end 150 107.5) (width 0.2) (layer "F.Cu") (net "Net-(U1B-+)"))
 (segment (start 156 107) (end 150.5 107) (width 0.2) (layer "F.Cu") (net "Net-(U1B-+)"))
 (segment (start 148.5 108.5) (end 150 108.5) (width 0.2) (layer "F.Cu") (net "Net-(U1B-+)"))
 (segment (start 154.3625 104.475) (end 155.975 104.475) (width 0.2) (layer "F.Cu") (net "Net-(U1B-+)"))
 (segment (start 156.5 106.5) (end 156 107) (width 0.2) (layer "F.Cu") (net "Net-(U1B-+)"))
 (segment (start 156.5 105) (end 156.5 106.5) (width 0.2) (layer "F.Cu") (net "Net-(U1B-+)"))
 (segment (start 150.5 112) (end 150.5 111) (width 0.2) (layer "F.Cu") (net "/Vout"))
 (segment (start 151 112.5) (end 150.5 112) (width 0.2) (layer "F.Cu") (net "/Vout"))
 (segment (start 158.5 103.175) (end 154.3625 103.175) (width 0.2) (layer "F.Cu") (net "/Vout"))
 (segment (start 151 110.5) (end 152.5 110.5) (width 0.2) (layer "F.Cu") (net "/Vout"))
 (segment (start 152.5 109.5) (end 153 109.5) (width 0.2) (layer "F.Cu") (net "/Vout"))
 (segment (start 158.8125 103.175) (end 158.5 103.175) (width 0.2) (layer "F.Cu") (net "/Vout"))
 (segment (start 161 104.5) (end 160.1375 104.5) (width 0.2) (layer "F.Cu") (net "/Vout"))
 (segment (start 154 108.5) (end 154.5 108.5) (width 0.2) (layer "F.Cu") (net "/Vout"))
 (segment (start 158.5 111) (end 157 112.5) (width 0.2) (layer "F.Cu") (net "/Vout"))
 (segment (start 153 109.5) (end 154 108.5) (width 0.2) (layer "F.Cu") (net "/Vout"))
 (segment (start 153 110) (end 153 109.5) (width 0.2) (layer "F.Cu") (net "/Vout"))
 (segment (start 152.5 110.5) (end 153 110) (width 0.2) (layer "F.Cu") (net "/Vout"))
 (segment (start 160.1375 104.5) (end 158.8125 103.175) (width 0.2) (layer "F.Cu") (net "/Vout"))
 (segment (start 152.5 109.5) (end 152.5 108.65) (width 0.2) (layer "F.Cu") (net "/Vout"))
 (segment (start 150.5 111) (end 151 110.5) (width 0.2) (layer "F.Cu") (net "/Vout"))
 (segment (start 157 112.5) (end 151 112.5) (width 0.2) (layer "F.Cu") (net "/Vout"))
 (segment (start 158.5 103.175) (end 158.5 111) (width 0.2) (layer "F.Cu") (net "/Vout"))
 (segment (start 152.5 108.65) (end 152.65 108.5) (width 0.2) (layer "F.Cu") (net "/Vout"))
 (segment (start 154.5 110.675) (end 153.675 111.5) (width 0.2) (layer "F.Cu") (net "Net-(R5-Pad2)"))
 (segment (start 154.5 109.5) (end 154.5 110.675) (width 0.2) (layer "F.Cu") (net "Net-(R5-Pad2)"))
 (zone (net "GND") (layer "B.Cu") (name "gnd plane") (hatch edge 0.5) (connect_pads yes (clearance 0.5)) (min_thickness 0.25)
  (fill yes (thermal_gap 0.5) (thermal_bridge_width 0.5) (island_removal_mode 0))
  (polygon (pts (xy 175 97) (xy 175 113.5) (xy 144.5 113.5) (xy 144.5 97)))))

